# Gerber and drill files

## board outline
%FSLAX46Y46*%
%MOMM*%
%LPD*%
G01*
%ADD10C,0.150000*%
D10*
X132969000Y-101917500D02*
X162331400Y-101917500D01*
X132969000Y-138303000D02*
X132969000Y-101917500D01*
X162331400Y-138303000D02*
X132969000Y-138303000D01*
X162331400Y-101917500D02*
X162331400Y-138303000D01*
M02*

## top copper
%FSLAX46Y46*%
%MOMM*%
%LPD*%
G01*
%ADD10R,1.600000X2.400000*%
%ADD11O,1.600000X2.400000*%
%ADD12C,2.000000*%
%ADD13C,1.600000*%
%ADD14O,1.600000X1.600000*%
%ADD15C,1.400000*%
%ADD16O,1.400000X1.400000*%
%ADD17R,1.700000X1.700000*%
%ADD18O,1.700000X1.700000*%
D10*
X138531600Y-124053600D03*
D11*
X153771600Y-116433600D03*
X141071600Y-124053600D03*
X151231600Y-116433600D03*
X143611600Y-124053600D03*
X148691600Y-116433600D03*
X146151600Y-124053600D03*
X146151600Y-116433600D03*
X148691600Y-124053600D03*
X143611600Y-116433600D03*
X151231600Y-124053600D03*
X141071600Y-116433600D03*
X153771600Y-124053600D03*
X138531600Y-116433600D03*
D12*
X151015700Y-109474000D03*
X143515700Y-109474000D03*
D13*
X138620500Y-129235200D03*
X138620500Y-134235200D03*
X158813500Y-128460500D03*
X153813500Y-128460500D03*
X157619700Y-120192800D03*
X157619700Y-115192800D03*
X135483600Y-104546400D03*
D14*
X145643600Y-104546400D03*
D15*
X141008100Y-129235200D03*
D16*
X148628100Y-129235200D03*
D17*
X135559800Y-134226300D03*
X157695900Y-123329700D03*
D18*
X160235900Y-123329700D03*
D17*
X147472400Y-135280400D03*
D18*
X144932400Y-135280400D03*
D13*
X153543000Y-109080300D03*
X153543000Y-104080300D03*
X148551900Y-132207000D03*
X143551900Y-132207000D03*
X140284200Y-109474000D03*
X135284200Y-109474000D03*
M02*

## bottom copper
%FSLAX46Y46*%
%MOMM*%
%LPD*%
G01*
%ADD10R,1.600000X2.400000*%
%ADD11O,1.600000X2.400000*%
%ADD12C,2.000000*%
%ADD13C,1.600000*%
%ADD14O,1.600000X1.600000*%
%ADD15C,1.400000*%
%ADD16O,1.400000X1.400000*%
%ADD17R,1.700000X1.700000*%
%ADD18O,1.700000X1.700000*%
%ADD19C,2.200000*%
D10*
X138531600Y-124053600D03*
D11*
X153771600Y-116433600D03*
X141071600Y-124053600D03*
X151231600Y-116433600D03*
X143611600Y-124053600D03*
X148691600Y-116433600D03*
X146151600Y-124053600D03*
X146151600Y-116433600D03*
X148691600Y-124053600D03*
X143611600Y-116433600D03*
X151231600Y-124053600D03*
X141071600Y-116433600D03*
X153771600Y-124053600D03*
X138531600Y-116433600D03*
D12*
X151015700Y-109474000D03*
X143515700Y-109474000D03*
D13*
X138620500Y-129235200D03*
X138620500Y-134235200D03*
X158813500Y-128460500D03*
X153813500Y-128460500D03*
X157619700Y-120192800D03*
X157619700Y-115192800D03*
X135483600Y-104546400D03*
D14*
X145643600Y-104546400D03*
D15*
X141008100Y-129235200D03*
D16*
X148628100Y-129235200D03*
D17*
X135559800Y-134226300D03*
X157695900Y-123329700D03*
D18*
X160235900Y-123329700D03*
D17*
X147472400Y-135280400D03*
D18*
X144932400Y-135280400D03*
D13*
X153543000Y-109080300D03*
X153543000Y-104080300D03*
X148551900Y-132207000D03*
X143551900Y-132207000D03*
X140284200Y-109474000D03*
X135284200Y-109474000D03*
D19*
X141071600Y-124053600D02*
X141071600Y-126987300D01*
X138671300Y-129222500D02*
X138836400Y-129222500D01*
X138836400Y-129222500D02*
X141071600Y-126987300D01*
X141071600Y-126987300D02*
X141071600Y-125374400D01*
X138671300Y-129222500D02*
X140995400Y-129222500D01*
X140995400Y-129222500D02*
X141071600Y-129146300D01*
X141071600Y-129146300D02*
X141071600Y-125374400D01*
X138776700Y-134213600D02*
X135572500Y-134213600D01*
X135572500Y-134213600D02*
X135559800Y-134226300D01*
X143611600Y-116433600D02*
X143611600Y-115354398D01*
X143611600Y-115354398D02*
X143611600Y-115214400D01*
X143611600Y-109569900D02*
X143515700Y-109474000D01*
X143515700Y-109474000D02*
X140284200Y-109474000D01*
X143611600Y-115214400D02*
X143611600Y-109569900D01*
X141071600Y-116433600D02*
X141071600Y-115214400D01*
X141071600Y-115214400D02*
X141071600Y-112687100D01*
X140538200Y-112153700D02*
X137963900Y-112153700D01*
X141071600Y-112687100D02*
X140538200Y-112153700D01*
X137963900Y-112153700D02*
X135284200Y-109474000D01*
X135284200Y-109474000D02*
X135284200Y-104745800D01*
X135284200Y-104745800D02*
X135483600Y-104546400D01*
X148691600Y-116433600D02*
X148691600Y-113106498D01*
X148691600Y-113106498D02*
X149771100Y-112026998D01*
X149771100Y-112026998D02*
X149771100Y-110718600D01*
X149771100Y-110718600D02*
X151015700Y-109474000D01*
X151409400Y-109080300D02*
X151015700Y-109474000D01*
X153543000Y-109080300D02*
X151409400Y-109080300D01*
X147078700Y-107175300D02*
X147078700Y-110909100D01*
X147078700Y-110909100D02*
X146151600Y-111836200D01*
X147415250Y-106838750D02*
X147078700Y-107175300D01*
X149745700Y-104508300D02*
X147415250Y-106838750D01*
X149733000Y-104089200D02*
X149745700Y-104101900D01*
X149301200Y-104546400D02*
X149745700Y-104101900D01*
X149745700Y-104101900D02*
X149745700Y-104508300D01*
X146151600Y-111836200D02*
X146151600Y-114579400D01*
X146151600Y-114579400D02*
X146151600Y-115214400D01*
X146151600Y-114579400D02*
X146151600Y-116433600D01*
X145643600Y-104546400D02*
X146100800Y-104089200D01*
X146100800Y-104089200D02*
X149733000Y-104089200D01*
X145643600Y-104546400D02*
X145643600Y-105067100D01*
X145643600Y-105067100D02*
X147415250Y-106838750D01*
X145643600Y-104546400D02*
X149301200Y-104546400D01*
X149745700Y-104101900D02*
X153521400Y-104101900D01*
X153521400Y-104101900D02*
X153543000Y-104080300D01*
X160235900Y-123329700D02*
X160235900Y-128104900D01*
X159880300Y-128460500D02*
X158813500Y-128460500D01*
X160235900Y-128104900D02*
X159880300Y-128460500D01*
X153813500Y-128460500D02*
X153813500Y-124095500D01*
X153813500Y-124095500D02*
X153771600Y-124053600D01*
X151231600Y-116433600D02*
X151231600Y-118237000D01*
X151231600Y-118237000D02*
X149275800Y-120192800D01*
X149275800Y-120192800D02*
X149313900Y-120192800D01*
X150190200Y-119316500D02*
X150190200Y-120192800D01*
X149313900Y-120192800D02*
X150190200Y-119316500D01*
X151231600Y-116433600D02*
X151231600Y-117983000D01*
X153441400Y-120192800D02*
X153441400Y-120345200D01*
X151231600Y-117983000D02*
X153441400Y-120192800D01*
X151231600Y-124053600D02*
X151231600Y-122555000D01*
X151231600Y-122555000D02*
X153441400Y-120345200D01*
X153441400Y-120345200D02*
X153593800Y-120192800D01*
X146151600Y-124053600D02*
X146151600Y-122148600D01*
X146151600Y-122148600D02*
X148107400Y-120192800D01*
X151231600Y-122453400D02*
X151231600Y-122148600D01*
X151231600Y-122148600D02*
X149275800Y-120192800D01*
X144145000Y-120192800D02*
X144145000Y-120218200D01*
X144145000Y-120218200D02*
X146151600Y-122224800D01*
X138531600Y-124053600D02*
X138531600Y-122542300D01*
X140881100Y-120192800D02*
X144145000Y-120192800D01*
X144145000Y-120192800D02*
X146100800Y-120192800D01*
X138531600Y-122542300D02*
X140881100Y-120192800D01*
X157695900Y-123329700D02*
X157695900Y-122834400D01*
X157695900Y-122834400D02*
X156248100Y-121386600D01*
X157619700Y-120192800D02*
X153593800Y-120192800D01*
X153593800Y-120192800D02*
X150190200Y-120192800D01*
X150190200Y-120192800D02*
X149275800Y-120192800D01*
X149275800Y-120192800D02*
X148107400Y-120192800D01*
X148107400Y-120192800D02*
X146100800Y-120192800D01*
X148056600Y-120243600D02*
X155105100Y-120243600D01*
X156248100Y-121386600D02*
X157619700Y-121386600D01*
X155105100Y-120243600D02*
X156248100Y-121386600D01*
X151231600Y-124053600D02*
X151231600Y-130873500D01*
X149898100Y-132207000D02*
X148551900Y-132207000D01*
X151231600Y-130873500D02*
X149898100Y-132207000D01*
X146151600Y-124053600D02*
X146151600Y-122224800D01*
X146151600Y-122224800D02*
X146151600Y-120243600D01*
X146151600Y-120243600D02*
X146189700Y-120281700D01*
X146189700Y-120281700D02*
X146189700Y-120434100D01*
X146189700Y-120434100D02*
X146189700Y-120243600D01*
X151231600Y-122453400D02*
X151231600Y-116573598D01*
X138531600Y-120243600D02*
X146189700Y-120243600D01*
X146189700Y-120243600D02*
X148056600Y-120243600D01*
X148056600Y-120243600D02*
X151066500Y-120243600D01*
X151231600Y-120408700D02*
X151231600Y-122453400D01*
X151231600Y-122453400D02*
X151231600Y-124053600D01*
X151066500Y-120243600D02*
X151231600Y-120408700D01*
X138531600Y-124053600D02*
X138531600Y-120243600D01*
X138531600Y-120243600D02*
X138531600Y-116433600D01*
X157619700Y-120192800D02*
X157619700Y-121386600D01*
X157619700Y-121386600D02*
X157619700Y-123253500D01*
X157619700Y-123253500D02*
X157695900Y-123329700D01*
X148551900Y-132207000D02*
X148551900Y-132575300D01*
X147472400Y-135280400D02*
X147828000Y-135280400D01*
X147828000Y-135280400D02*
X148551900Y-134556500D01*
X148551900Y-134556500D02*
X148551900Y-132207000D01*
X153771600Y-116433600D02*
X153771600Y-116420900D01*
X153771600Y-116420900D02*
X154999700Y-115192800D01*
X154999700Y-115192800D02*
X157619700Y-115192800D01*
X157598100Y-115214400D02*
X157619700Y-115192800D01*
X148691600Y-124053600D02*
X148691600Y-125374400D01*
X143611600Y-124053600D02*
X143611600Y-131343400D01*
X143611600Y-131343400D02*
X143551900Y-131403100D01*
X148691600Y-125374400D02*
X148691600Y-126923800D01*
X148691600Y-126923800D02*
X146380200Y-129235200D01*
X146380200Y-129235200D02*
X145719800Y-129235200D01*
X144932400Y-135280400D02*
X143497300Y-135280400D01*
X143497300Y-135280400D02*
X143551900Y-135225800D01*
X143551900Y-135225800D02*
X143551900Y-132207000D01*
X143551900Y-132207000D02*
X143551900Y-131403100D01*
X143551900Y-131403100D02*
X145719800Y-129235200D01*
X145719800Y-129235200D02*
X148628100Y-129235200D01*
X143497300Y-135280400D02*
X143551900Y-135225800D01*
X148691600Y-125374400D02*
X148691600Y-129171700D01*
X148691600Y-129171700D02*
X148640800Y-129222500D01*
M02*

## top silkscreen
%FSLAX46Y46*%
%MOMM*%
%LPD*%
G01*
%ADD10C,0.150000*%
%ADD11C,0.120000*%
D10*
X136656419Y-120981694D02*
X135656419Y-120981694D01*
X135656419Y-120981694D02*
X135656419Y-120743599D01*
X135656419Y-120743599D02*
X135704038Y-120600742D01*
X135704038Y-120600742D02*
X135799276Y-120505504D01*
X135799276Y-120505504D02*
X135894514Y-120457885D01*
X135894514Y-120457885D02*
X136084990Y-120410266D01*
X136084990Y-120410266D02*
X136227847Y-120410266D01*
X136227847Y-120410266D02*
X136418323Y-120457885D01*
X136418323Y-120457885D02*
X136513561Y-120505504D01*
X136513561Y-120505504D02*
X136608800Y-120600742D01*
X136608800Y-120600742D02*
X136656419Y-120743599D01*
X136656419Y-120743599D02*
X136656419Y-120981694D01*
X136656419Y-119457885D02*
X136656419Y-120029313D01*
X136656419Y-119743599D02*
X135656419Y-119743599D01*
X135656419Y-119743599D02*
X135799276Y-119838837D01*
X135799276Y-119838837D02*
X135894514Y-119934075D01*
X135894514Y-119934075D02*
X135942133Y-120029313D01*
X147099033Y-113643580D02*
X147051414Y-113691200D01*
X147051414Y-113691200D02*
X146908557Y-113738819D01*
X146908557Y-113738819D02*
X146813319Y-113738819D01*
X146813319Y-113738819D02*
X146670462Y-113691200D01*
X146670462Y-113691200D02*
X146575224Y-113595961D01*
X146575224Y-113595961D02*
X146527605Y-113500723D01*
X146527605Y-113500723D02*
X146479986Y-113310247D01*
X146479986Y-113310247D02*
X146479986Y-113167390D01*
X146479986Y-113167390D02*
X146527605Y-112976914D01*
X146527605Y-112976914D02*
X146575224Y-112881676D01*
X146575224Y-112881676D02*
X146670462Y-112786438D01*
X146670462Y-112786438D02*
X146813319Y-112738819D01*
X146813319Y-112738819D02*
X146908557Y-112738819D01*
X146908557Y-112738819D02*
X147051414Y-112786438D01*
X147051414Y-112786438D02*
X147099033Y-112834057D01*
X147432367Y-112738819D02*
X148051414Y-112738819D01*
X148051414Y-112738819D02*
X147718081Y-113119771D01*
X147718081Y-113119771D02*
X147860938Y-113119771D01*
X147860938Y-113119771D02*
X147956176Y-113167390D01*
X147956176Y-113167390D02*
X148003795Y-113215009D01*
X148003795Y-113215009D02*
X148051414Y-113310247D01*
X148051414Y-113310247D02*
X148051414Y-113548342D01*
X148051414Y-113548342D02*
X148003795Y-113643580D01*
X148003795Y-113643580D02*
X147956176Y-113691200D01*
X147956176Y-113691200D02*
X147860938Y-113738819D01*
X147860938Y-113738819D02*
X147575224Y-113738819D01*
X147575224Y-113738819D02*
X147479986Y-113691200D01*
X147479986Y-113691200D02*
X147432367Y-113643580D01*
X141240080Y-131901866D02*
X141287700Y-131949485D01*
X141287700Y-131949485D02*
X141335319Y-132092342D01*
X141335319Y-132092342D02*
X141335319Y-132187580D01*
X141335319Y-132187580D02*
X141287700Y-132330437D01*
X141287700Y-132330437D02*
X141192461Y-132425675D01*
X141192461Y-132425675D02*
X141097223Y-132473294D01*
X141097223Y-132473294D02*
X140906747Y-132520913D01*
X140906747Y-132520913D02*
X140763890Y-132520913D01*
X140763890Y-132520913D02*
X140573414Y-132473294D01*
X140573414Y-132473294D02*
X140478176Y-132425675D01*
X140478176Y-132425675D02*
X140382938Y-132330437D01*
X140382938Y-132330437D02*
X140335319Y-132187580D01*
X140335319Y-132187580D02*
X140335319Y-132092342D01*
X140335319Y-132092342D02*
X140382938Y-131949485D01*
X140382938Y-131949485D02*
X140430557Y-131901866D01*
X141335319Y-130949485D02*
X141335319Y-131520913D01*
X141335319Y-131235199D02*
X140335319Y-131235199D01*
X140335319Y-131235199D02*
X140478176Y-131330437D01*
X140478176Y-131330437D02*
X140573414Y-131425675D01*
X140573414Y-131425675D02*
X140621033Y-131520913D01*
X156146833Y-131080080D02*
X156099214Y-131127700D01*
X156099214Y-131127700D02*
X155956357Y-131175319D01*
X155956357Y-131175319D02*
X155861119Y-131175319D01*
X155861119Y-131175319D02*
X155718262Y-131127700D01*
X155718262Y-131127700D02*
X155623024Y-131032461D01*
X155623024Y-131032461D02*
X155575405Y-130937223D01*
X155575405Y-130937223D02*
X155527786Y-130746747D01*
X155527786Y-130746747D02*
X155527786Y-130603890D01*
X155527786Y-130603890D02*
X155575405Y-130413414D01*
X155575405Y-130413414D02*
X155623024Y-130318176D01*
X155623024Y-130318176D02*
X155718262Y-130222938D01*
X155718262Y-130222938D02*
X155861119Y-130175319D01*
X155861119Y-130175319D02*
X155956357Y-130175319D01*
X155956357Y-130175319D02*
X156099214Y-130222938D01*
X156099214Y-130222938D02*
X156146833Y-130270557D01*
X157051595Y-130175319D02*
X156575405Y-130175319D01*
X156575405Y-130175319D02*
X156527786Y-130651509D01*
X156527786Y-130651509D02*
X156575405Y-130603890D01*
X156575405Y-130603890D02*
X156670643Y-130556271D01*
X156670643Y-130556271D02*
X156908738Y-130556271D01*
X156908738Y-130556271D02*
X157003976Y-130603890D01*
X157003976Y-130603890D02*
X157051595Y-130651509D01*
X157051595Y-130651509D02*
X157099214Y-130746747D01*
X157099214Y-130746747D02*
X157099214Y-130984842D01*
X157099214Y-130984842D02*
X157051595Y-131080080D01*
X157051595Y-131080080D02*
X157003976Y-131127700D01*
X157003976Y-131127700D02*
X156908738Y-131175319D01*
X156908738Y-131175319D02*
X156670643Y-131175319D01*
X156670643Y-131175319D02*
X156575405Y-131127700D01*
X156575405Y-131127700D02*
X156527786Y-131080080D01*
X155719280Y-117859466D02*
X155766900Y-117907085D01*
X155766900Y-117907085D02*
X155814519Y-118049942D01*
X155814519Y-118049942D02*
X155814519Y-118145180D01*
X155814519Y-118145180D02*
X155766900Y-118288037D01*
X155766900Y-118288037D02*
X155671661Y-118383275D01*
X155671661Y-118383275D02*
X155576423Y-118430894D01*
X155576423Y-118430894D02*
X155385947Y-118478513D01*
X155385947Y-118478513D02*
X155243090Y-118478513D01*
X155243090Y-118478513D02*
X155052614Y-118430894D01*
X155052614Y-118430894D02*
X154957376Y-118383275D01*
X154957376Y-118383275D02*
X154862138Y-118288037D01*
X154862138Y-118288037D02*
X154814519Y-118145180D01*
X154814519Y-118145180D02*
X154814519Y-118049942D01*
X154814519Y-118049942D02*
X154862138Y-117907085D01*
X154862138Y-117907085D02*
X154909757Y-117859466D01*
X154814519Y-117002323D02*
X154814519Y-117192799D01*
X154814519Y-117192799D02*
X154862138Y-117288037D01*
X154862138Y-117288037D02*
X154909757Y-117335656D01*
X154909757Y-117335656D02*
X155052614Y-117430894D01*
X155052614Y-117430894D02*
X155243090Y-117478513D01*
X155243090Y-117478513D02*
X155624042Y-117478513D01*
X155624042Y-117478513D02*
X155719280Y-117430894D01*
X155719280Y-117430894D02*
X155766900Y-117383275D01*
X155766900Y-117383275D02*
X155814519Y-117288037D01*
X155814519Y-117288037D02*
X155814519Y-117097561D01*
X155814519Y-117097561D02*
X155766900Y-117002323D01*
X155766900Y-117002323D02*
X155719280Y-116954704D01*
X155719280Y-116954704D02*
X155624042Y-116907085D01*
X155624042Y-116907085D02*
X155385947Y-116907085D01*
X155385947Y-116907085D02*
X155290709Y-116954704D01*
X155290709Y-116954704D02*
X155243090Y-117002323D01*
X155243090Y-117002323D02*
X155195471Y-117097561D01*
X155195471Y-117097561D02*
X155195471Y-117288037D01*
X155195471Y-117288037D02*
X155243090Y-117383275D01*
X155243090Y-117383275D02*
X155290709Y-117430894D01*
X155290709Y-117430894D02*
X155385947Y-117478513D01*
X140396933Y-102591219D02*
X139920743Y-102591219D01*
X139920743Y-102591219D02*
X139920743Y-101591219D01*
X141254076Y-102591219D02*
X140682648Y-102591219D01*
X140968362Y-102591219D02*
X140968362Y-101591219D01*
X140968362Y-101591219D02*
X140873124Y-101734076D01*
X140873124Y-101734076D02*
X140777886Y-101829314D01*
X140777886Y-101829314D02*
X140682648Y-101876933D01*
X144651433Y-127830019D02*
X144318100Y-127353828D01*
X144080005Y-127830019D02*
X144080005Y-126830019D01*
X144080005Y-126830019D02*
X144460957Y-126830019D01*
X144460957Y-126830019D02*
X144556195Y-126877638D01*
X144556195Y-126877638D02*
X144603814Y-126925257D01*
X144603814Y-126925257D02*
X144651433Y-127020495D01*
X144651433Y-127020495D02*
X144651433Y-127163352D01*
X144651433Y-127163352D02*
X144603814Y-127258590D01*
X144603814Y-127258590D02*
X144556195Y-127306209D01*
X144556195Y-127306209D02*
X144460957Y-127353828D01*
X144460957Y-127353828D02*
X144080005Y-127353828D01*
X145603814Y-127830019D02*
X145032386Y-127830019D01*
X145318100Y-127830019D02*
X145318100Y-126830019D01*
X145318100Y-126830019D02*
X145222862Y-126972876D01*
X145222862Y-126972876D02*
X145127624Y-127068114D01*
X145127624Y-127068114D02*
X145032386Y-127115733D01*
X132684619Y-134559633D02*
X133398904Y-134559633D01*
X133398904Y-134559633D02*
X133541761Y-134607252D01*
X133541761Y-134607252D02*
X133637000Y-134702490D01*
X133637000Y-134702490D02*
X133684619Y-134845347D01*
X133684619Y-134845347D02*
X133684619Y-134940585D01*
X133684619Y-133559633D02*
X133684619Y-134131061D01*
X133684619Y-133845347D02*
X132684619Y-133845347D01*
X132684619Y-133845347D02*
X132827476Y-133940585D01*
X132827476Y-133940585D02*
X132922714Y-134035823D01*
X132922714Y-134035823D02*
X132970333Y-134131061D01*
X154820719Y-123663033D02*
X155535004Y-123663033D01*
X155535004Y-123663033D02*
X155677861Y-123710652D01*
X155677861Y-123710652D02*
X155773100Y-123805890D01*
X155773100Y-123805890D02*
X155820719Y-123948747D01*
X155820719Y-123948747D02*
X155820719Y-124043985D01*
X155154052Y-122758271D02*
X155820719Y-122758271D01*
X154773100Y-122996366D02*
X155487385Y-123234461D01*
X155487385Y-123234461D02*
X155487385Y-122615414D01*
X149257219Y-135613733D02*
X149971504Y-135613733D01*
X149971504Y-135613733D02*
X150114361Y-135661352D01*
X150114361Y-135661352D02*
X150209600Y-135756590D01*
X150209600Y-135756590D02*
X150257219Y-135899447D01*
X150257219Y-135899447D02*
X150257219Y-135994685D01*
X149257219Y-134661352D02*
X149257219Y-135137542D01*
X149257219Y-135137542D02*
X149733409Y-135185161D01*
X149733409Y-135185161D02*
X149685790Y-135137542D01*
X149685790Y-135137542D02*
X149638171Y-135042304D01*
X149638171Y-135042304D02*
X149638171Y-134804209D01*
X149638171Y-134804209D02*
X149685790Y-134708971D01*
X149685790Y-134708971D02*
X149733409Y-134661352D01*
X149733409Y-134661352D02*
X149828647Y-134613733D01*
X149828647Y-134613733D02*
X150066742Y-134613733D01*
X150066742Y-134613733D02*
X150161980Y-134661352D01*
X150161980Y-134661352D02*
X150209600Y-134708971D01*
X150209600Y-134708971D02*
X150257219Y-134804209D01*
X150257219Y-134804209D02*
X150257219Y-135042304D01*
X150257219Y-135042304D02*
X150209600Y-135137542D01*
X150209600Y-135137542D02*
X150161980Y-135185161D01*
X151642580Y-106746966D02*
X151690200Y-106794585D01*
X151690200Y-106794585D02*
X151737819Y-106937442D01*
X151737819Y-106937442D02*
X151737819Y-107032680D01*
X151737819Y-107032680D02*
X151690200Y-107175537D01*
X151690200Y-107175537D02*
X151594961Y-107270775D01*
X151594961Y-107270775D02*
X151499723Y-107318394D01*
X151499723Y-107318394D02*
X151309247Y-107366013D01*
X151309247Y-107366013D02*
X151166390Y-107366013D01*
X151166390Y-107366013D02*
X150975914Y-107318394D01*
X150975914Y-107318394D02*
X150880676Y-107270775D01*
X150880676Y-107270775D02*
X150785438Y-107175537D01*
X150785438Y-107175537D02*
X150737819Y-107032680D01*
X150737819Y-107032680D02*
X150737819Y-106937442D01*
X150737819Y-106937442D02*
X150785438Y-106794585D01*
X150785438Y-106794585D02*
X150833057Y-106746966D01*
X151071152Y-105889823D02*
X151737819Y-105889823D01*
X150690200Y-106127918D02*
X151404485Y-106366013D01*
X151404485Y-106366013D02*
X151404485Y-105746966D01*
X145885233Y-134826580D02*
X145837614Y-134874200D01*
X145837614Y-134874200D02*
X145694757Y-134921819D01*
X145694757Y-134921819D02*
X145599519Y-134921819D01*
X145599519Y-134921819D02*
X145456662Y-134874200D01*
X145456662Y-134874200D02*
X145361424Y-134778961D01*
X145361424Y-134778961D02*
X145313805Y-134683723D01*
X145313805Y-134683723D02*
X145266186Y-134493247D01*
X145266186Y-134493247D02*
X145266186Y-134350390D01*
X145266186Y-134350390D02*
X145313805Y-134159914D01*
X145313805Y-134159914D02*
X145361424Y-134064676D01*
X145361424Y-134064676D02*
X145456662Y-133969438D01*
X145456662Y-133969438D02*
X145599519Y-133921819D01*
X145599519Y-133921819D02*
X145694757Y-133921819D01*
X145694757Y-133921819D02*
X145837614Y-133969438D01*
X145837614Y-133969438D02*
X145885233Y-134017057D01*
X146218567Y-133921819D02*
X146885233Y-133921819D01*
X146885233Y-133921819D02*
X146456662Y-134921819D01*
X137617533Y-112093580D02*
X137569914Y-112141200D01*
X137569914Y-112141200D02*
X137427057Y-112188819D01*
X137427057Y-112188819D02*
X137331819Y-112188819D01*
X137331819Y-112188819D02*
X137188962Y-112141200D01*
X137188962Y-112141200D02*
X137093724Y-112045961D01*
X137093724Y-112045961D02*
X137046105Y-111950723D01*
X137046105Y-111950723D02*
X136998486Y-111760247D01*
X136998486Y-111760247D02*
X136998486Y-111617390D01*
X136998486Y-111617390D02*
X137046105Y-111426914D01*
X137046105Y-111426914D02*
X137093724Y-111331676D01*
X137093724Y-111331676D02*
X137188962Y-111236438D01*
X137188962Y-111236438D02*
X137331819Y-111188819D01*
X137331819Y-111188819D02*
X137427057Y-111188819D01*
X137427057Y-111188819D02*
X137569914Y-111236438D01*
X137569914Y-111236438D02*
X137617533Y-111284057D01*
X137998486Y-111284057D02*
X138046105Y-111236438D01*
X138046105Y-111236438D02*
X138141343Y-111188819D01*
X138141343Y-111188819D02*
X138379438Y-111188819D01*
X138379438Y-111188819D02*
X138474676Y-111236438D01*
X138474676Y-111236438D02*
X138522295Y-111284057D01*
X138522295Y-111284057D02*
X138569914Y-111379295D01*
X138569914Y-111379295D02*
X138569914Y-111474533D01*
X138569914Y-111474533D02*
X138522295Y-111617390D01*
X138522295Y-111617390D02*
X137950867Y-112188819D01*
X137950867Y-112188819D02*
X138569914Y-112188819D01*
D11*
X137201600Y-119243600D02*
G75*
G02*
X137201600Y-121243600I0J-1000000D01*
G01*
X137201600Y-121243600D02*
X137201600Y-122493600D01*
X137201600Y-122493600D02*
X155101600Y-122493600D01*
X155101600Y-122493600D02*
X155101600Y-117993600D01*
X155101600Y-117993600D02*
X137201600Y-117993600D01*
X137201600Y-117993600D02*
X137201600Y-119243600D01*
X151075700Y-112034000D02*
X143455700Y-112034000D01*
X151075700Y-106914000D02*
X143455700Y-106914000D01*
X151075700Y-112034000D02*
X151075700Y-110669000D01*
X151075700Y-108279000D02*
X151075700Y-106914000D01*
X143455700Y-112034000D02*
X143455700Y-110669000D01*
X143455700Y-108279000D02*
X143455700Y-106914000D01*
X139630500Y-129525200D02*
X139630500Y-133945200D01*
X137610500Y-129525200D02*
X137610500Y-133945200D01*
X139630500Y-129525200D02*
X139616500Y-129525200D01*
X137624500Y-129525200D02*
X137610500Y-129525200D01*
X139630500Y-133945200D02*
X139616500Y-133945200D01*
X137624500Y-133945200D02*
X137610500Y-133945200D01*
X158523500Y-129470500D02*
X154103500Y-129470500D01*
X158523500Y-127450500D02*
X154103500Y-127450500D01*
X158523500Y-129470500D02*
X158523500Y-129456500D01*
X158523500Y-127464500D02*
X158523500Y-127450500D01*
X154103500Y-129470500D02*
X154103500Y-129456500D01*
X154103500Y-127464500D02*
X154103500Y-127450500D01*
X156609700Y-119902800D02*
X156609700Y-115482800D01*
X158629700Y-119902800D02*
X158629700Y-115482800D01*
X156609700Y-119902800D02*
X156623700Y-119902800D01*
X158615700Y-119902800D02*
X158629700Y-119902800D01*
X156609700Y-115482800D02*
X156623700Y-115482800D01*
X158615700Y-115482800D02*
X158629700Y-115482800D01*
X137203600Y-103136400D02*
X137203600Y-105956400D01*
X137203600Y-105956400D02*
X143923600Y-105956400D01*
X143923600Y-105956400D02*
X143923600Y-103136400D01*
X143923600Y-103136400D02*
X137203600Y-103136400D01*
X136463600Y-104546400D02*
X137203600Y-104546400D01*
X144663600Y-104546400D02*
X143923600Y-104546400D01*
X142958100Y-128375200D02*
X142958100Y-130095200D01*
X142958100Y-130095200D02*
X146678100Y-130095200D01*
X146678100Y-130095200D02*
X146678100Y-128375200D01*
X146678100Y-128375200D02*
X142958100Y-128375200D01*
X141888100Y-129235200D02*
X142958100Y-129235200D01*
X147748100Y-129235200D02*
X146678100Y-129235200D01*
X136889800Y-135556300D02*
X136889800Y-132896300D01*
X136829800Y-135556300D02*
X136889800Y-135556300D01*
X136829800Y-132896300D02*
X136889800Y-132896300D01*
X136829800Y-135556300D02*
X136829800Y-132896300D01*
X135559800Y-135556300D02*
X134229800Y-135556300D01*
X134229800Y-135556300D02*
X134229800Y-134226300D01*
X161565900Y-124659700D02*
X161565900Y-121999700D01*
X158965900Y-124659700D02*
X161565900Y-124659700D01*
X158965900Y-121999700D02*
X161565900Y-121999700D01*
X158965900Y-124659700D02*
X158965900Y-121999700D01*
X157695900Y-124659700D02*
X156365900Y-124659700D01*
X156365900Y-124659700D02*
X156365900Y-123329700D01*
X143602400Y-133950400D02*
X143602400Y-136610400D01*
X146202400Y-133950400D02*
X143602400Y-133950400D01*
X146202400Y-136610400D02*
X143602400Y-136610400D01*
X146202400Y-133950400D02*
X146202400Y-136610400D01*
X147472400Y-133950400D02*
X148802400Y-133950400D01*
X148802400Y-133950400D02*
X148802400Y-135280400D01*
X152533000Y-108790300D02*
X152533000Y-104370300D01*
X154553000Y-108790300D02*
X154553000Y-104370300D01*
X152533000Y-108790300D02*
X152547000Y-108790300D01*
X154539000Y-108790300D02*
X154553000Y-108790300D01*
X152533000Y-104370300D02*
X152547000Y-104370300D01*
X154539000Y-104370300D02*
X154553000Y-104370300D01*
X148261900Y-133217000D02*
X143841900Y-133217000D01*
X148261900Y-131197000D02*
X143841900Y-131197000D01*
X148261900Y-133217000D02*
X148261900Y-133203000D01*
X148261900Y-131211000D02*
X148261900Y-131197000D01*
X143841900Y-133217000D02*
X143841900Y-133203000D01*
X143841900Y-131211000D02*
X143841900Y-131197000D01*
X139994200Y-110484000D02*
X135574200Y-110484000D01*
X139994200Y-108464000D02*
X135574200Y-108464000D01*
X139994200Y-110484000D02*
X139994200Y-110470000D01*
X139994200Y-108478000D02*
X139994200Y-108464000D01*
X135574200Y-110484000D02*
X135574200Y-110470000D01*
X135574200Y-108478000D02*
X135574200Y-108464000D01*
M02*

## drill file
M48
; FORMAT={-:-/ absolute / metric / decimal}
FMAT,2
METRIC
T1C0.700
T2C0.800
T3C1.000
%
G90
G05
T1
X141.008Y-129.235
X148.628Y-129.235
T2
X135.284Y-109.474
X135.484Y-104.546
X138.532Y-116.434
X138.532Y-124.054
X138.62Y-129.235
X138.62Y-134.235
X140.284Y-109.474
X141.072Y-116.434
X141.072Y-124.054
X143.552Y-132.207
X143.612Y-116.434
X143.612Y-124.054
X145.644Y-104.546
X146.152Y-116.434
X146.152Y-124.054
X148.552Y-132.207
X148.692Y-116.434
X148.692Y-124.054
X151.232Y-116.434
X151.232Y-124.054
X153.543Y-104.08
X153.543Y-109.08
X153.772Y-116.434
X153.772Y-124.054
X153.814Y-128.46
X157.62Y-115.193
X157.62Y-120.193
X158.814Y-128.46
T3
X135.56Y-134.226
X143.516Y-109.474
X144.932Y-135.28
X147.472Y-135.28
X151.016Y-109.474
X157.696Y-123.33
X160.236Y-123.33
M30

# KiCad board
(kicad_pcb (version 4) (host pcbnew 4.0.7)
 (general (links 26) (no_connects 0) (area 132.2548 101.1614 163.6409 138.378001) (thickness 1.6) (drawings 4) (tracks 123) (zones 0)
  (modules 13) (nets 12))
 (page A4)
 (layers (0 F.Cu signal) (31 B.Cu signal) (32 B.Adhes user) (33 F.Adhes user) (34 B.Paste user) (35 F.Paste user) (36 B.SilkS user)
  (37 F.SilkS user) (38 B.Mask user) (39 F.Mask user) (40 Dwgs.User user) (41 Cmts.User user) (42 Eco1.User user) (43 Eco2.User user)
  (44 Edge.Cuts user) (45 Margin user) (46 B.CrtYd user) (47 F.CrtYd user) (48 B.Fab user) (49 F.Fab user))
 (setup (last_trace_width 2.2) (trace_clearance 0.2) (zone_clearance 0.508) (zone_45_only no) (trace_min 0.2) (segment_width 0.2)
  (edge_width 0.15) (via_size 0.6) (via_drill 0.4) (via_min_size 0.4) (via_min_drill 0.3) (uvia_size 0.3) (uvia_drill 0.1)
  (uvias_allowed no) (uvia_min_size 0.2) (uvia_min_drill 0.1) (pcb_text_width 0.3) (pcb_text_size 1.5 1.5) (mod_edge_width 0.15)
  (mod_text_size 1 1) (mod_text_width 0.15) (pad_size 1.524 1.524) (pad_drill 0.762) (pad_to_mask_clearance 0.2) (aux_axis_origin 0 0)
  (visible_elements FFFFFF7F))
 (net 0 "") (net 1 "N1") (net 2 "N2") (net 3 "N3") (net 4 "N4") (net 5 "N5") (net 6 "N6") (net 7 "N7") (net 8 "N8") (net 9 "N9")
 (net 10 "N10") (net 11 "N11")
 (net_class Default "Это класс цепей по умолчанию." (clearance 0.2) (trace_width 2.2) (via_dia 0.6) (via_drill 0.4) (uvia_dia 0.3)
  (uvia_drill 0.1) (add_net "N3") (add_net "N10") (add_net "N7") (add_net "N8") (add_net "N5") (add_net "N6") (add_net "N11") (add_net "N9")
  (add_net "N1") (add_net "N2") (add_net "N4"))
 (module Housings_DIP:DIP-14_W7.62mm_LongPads (layer F.Cu) (at 138.5316 124.0536 90)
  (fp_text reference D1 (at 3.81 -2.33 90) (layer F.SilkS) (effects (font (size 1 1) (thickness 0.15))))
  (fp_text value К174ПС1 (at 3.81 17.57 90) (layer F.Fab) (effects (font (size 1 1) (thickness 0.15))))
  (fp_arc (start 3.81 -1.33) (end 2.81 -1.33) (angle -180) (layer F.SilkS) (width 0.12))
  (fp_line (start 2.81 -1.33) (end 1.56 -1.33) (layer F.SilkS) (width 0.12))
  (fp_line (start 1.56 -1.33) (end 1.56 16.57) (layer F.SilkS) (width 0.12))
  (fp_line (start 1.56 16.57) (end 6.06 16.57) (layer F.SilkS) (width 0.12))
  (fp_line (start 6.06 16.57) (end 6.06 -1.33) (layer F.SilkS) (width 0.12))
  (fp_line (start 6.06 -1.33) (end 4.81 -1.33) (layer F.SilkS) (width 0.12))
  (pad 1 thru_hole rect (at 0 0 90) (size 2.4 1.6) (drill 0.8) (layers *.Cu *.Mask) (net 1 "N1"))
  (pad 8 thru_hole oval (at 7.62 15.24 90) (size 2.4 1.6) (drill 0.8) (layers *.Cu *.Mask) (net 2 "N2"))
  (pad 2 thru_hole oval (at 0 2.54 90) (size 2.4 1.6) (drill 0.8) (layers *.Cu *.Mask) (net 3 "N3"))
  (pad 9 thru_hole oval (at 7.62 12.7 90) (size 2.4 1.6) (drill 0.8) (layers *.Cu *.Mask) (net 1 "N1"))
  (pad 3 thru_hole oval (at 0 5.08 90) (size 2.4 1.6) (drill 0.8) (layers *.Cu *.Mask) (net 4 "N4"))
  (pad 10 thru_hole oval (at 7.62 10.16 90) (size 2.4 1.6) (drill 0.8) (layers *.Cu *.Mask) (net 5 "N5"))
  (pad 4 thru_hole oval (at 0 7.62 90) (size 2.4 1.6) (drill 0.8) (layers *.Cu *.Mask) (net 1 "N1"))
  (pad 11 thru_hole oval (at 7.62 7.62 90) (size 2.4 1.6) (drill 0.8) (layers *.Cu *.Mask) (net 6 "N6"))
  (pad 5 thru_hole oval (at 0 10.16 90) (size 2.4 1.6) (drill 0.8) (layers *.Cu *.Mask) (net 4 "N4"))
  (pad 12 thru_hole oval (at 7.62 5.08 90) (size 2.4 1.6) (drill 0.8) (layers *.Cu *.Mask) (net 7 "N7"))
  (pad 6 thru_hole oval (at 0 12.7 90) (size 2.4 1.6) (drill 0.8) (layers *.Cu *.Mask) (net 1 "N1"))
  (pad 13 thru_hole oval (at 7.62 2.54 90) (size 2.4 1.6) (drill 0.8) (layers *.Cu *.Mask) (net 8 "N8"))
  (pad 7 thru_hole oval (at 0 15.24 90) (size 2.4 1.6) (drill 0.8) (layers *.Cu *.Mask) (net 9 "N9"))
  (pad 14 thru_hole oval (at 7.62 0 90) (size 2.4 1.6) (drill 0.8) (layers *.Cu *.Mask) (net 1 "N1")))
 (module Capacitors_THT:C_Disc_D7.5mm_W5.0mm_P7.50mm (layer F.Cu) (at 151.0157 109.474 180)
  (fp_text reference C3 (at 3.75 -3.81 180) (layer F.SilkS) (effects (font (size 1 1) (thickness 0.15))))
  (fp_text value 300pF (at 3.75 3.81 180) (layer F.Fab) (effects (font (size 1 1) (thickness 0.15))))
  (fp_line (start -0.06 -2.56) (end 7.56 -2.56) (layer F.SilkS) (width 0.12))
  (fp_line (start -0.06 2.56) (end 7.56 2.56) (layer F.SilkS) (width 0.12))
  (fp_line (start -0.06 -2.56) (end -0.06 -1.195) (layer F.SilkS) (width 0.12))
  (fp_line (start -0.06 1.195) (end -0.06 2.56) (layer F.SilkS) (width 0.12))
  (fp_line (start 7.56 -2.56) (end 7.56 -1.195) (layer F.SilkS) (width 0.12))
  (fp_line (start 7.56 1.195) (end 7.56 2.56) (layer F.SilkS) (width 0.12))
  (pad 1 thru_hole circle (at 0 0 180) (size 2 2) (drill 1) (layers *.Cu *.Mask) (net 5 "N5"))
  (pad 2 thru_hole circle (at 7.5 0 180) (size 2 2) (drill 1) (layers *.Cu *.Mask) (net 7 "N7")))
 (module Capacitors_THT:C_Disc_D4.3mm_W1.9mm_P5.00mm (layer F.Cu) (at 138.6205 129.2352 270)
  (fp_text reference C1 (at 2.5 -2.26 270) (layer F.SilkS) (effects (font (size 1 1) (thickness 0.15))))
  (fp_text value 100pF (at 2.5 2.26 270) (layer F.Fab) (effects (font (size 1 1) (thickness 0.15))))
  (fp_line (start 0.29 -1.01) (end 4.71 -1.01) (layer F.SilkS) (width 0.12))
  (fp_line (start 0.29 1.01) (end 4.71 1.01) (layer F.SilkS) (width 0.12))
  (fp_line (start 0.29 -1.01) (end 0.29 -0.996) (layer F.SilkS) (width 0.12))
  (fp_line (start 0.29 0.996) (end 0.29 1.01) (layer F.SilkS) (width 0.12))
  (fp_line (start 4.71 -1.01) (end 4.71 -0.996) (layer F.SilkS) (width 0.12))
  (fp_line (start 4.71 0.996) (end 4.71 1.01) (layer F.SilkS) (width 0.12))
  (pad 1 thru_hole circle (at 0 0 270) (size 1.6 1.6) (drill 0.8) (layers *.Cu *.Mask) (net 3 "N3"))
  (pad 2 thru_hole circle (at 5 0 270) (size 1.6 1.6) (drill 0.8) (layers *.Cu *.Mask) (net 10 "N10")))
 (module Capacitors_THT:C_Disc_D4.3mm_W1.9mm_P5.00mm (layer F.Cu) (at 158.8135 128.4605 180)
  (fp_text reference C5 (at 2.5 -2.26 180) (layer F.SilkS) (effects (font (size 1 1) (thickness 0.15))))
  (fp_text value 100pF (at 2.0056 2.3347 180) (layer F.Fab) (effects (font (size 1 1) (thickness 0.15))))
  (fp_line (start 0.29 -1.01) (end 4.71 -1.01) (layer F.SilkS) (width 0.12))
  (fp_line (start 0.29 1.01) (end 4.71 1.01) (layer F.SilkS) (width 0.12))
  (fp_line (start 0.29 -1.01) (end 0.29 -0.996) (layer F.SilkS) (width 0.12))
  (fp_line (start 0.29 0.996) (end 0.29 1.01) (layer F.SilkS) (width 0.12))
  (fp_line (start 4.71 -1.01) (end 4.71 -0.996) (layer F.SilkS) (width 0.12))
  (fp_line (start 4.71 0.996) (end 4.71 1.01) (layer F.SilkS) (width 0.12))
  (pad 1 thru_hole circle (at 0 0 180) (size 1.6 1.6) (drill 0.8) (layers *.Cu *.Mask) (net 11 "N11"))
  (pad 2 thru_hole circle (at 5 0 180) (size 1.6 1.6) (drill 0.8) (layers *.Cu *.Mask) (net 9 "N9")))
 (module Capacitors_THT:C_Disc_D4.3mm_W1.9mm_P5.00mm (layer F.Cu) (at 157.6197 120.1928 90)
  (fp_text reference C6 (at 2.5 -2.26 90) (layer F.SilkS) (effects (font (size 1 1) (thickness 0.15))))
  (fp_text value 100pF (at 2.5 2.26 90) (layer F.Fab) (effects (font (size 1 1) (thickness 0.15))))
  (fp_line (start 0.29 -1.01) (end 4.71 -1.01) (layer F.SilkS) (width 0.12))
  (fp_line (start 0.29 1.01) (end 4.71 1.01) (layer F.SilkS) (width 0.12))
  (fp_line (start 0.29 -1.01) (end 0.29 -0.996) (layer F.SilkS) (width 0.12))
  (fp_line (start 0.29 0.996) (end 0.29 1.01) (layer F.SilkS) (width 0.12))
  (fp_line (start 4.71 -1.01) (end 4.71 -0.996) (layer F.SilkS) (width 0.12))
  (fp_line (start 4.71 0.996) (end 4.71 1.01) (layer F.SilkS) (width 0.12))
  (pad 1 thru_hole circle (at 0 0 90) (size 1.6 1.6) (drill 0.8) (layers *.Cu *.Mask) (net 1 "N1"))
  (pad 2 thru_hole circle (at 5 0 90) (size 1.6 1.6) (drill 0.8) (layers *.Cu *.Mask) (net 2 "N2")))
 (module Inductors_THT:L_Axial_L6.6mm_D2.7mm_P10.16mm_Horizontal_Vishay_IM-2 (layer F.Cu) (at 135.4836 104.5464)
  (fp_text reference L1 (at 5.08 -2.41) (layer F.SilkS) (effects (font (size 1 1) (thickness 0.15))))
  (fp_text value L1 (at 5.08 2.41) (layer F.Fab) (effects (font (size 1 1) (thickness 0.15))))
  (fp_line (start 1.72 -1.41) (end 1.72 1.41) (layer F.SilkS) (width 0.12))
  (fp_line (start 1.72 1.41) (end 8.44 1.41) (layer F.SilkS) (width 0.12))
  (fp_line (start 8.44 1.41) (end 8.44 -1.41) (layer F.SilkS) (width 0.12))
  (fp_line (start 8.44 -1.41) (end 1.72 -1.41) (layer F.SilkS) (width 0.12))
  (fp_line (start 0.98 0) (end 1.72 0) (layer F.SilkS) (width 0.12))
  (fp_line (start 9.18 0) (end 8.44 0) (layer F.SilkS) (width 0.12))
  (pad 1 thru_hole circle (at 0 0) (size 1.6 1.6) (drill 0.8) (layers *.Cu *.Mask) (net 8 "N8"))
  (pad 2 thru_hole oval (at 10.16 0) (size 1.6 1.6) (drill 0.8) (layers *.Cu *.Mask) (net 6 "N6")))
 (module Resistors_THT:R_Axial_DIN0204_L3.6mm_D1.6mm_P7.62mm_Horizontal (layer F.Cu) (at 141.0081 129.2352)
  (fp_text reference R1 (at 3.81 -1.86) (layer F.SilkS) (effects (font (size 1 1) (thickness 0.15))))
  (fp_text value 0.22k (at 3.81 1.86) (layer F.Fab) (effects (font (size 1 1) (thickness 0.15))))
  (fp_line (start 1.95 -0.86) (end 1.95 0.86) (layer F.SilkS) (width 0.12))
  (fp_line (start 1.95 0.86) (end 5.67 0.86) (layer F.SilkS) (width 0.12))
  (fp_line (start 5.67 0.86) (end 5.67 -0.86) (layer F.SilkS) (width 0.12))
  (fp_line (start 5.67 -0.86) (end 1.95 -0.86) (layer F.SilkS) (width 0.12))
  (fp_line (start 0.88 0) (end 1.95 0) (layer F.SilkS) (width 0.12))
  (fp_line (start 6.74 0) (end 5.67 0) (layer F.SilkS) (width 0.12))
  (pad 1 thru_hole circle (at 0 0) (size 1.4 1.4) (drill 0.7) (layers *.Cu *.Mask) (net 3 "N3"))
  (pad 2 thru_hole oval (at 7.62 0) (size 1.4 1.4) (drill 0.7) (layers *.Cu *.Mask) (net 4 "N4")))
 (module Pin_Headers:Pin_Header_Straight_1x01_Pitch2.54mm (layer F.Cu) (at 135.5598 134.2263 90)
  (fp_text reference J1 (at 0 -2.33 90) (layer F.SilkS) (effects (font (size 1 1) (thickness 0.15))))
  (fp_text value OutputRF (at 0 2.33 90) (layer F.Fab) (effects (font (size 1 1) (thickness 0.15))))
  (fp_line (start -1.33 1.33) (end 1.33 1.33) (layer F.SilkS) (width 0.12))
  (fp_line (start -1.33 1.27) (end -1.33 1.33) (layer F.SilkS) (width 0.12))
  (fp_line (start 1.33 1.27) (end 1.33 1.33) (layer F.SilkS) (width 0.12))
  (fp_line (start -1.33 1.27) (end 1.33 1.27) (layer F.SilkS) (width 0.12))
  (fp_line (start -1.33 0) (end -1.33 -1.33) (layer F.SilkS) (width 0.12))
  (fp_line (start -1.33 -1.33) (end 0 -1.33) (layer F.SilkS) (width 0.12))
  (pad 1 thru_hole rect (at 0 0 90) (size 1.7 1.7) (drill 1) (layers *.Cu *.Mask) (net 10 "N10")))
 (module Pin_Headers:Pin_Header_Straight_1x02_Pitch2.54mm (layer F.Cu) (at 157.6959 123.3297 90)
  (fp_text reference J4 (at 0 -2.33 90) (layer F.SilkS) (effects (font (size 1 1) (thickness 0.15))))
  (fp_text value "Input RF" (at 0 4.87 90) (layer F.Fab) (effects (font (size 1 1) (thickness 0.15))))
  (fp_line (start -1.33 3.87) (end 1.33 3.87) (layer F.SilkS) (width 0.12))
  (fp_line (start -1.33 1.27) (end -1.33 3.87) (layer F.SilkS) (width 0.12))
  (fp_line (start 1.33 1.27) (end 1.33 3.87) (layer F.SilkS) (width 0.12))
  (fp_line (start -1.33 1.27) (end 1.33 1.27) (layer F.SilkS) (width 0.12))
  (fp_line (start -1.33 0) (end -1.33 -1.33) (layer F.SilkS) (width 0.12))
  (fp_line (start -1.33 -1.33) (end 0 -1.33) (layer F.SilkS) (width 0.12))
  (pad 1 thru_hole rect (at 0 0 90) (size 1.7 1.7) (drill 1) (layers *.Cu *.Mask) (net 1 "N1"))
  (pad 2 thru_hole oval (at 0 2.54 90) (size 1.7 1.7) (drill 1) (layers *.Cu *.Mask) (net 11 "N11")))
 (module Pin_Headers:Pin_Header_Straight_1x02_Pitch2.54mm (layer F.Cu) (at 147.4724 135.2804 270)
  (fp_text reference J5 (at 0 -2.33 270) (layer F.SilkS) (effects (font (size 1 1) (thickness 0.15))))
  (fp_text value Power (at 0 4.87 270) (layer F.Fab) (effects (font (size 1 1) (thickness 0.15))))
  (fp_line (start -1.33 3.87) (end 1.33 3.87) (layer F.SilkS) (width 0.12))
  (fp_line (start -1.33 1.27) (end -1.33 3.87) (layer F.SilkS) (width 0.12))
  (fp_line (start 1.33 1.27) (end 1.33 3.87) (layer F.SilkS) (width 0.12))
  (fp_line (start -1.33 1.27) (end 1.33 1.27) (layer F.SilkS) (width 0.12))
  (fp_line (start -1.33 0) (end -1.33 -1.33) (layer F.SilkS) (width 0.12))
  (fp_line (start -1.33 -1.33) (end 0 -1.33) (layer F.SilkS) (width 0.12))
  (pad 1 thru_hole rect (at 0 0 270) (size 1.7 1.7) (drill 1) (layers *.Cu *.Mask) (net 1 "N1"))
  (pad 2 thru_hole oval (at 0 2.54 270) (size 1.7 1.7) (drill 1) (layers *.Cu *.Mask) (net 4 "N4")))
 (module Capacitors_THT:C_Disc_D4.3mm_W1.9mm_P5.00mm (layer F.Cu) (at 153.543 109.0803 90)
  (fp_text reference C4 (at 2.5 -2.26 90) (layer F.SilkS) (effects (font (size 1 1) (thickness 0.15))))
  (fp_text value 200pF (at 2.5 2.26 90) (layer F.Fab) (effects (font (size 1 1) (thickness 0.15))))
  (fp_line (start 0.29 -1.01) (end 4.71 -1.01) (layer F.SilkS) (width 0.12))
  (fp_line (start 0.29 1.01) (end 4.71 1.01) (layer F.SilkS) (width 0.12))
  (fp_line (start 0.29 -1.01) (end 0.29 -0.996) (layer F.SilkS) (width 0.12))
  (fp_line (start 0.29 0.996) (end 0.29 1.01) (layer F.SilkS) (width 0.12))
  (fp_line (start 4.71 -1.01) (end 4.71 -0.996) (layer F.SilkS) (width 0.12))
  (fp_line (start 4.71 0.996) (end 4.71 1.01) (layer F.SilkS) (width 0.12))
  (pad 1 thru_hole circle (at 0 0 90) (size 1.6 1.6) (drill 0.8) (layers *.Cu *.Mask) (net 5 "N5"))
  (pad 2 thru_hole circle (at 5 0 90) (size 1.6 1.6) (drill 0.8) (layers *.Cu *.Mask) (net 6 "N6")))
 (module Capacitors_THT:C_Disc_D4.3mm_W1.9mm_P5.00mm (layer F.Cu) (at 148.5519 132.207 180)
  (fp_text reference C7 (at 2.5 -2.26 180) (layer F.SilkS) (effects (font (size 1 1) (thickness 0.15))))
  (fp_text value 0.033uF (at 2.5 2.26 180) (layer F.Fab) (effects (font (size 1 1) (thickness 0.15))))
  (fp_line (start 0.29 -1.01) (end 4.71 -1.01) (layer F.SilkS) (width 0.12))
  (fp_line (start 0.29 1.01) (end 4.71 1.01) (layer F.SilkS) (width 0.12))
  (fp_line (start 0.29 -1.01) (end 0.29 -0.996) (layer F.SilkS) (width 0.12))
  (fp_line (start 0.29 0.996) (end 0.29 1.01) (layer F.SilkS) (width 0.12))
  (fp_line (start 4.71 -1.01) (end 4.71 -0.996) (layer F.SilkS) (width 0.12))
  (fp_line (start 4.71 0.996) (end 4.71 1.01) (layer F.SilkS) (width 0.12))
  (pad 1 thru_hole circle (at 0 0 180) (size 1.6 1.6) (drill 0.8) (layers *.Cu *.Mask) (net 1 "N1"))
  (pad 2 thru_hole circle (at 5 0 180) (size 1.6 1.6) (drill 0.8) (layers *.Cu *.Mask) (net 4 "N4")))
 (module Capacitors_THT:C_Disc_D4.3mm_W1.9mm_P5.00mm (layer F.Cu) (at 140.2842 109.474 180)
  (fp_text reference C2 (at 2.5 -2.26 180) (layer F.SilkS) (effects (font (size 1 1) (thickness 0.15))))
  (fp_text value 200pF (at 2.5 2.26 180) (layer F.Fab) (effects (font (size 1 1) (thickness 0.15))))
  (fp_line (start 0.29 -1.01) (end 4.71 -1.01) (layer F.SilkS) (width 0.12))
  (fp_line (start 0.29 1.01) (end 4.71 1.01) (layer F.SilkS) (width 0.12))
  (fp_line (start 0.29 -1.01) (end 0.29 -0.996) (layer F.SilkS) (width 0.12))
  (fp_line (start 0.29 0.996) (end 0.29 1.01) (layer F.SilkS) (width 0.12))
  (fp_line (start 4.71 -1.01) (end 4.71 -0.996) (layer F.SilkS) (width 0.12))
  (fp_line (start 4.71 0.996) (end 4.71 1.01) (layer F.SilkS) (width 0.12))
  (pad 1 thru_hole circle (at 0 0 180) (size 1.6 1.6) (drill 0.8) (layers *.Cu *.Mask) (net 7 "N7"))
  (pad 2 thru_hole circle (at 5 0 180) (size 1.6 1.6) (drill 0.8) (layers *.Cu *.Mask) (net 8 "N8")))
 (gr_line (start 132.969 101.9175) (end 162.3314 101.9175) (angle 90) (layer Edge.Cuts) (width 0.15))
 (gr_line (start 132.969 138.303) (end 132.969 101.9175) (angle 90) (layer Edge.Cuts) (width 0.15))
 (gr_line (start 162.3314 138.303) (end 132.969 138.303) (angle 90) (layer Edge.Cuts) (width 0.15))
 (gr_line (start 162.3314 101.9175) (end 162.3314 138.303) (angle 90) (layer Edge.Cuts) (width 0.15))
 (segment (start 141.0716 124.0536) (end 141.0716 126.9873) (width 2.2) (layer B.Cu) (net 3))
 (segment (start 138.6713 129.2225) (end 138.8364 129.2225) (width 2.2) (layer B.Cu) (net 3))
 (segment (start 138.8364 129.2225) (end 141.0716 126.9873) (width 2.2) (layer B.Cu) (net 3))
 (segment (start 141.0716 126.9873) (end 141.0716 125.3744) (width 2.2) (layer B.Cu) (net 3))
 (segment (start 138.6713 129.2225) (end 140.9954 129.2225) (width 2.2) (layer B.Cu) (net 3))
 (segment (start 140.9954 129.2225) (end 141.0716 129.1463) (width 2.2) (layer B.Cu) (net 3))
 (segment (start 141.0716 129.1463) (end 141.0716 125.3744) (width 2.2) (layer B.Cu) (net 3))
 (segment (start 138.7767 134.2136) (end 135.5725 134.2136) (width 2.2) (layer B.Cu) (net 10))
 (segment (start 135.5725 134.2136) (end 135.5598 134.2263) (width 2.2) (layer B.Cu) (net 10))
 (segment (start 143.6116 116.4336) (end 143.6116 115.354398) (width 2.2) (layer B.Cu) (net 7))
 (segment (start 143.6116 115.354398) (end 143.6116 115.2144) (width 2.2) (layer B.Cu) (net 7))
 (segment (start 143.6116 109.5699) (end 143.5157 109.474) (width 2.2) (layer B.Cu) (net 7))
 (segment (start 143.5157 109.474) (end 140.2842 109.474) (width 2.2) (layer B.Cu) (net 7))
 (segment (start 143.6116 115.2144) (end 143.6116 109.5699) (width 2.2) (layer B.Cu) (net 7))
 (segment (start 141.0716 116.4336) (end 141.0716 115.2144) (width 2.2) (layer B.Cu) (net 8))
 (segment (start 141.0716 115.2144) (end 141.0716 112.6871) (width 2.2) (layer B.Cu) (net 8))
 (segment (start 140.5382 112.1537) (end 137.9639 112.1537) (width 2.2) (layer B.Cu) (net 8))
 (segment (start 141.0716 112.6871) (end 140.5382 112.1537) (width 2.2) (layer B.Cu) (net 8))
 (segment (start 137.9639 112.1537) (end 135.2842 109.474) (width 2.2) (layer B.Cu) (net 8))
 (segment (start 135.2842 109.474) (end 135.2842 104.7458) (width 2.2) (layer B.Cu) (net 8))
 (segment (start 135.2842 104.7458) (end 135.4836 104.5464) (width 2.2) (layer B.Cu) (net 8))
 (segment (start 148.6916 116.4336) (end 148.6916 113.106498) (width 2.2) (layer B.Cu) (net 5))
 (segment (start 148.6916 113.106498) (end 149.7711 112.026998) (width 2.2) (layer B.Cu) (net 5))
 (segment (start 149.7711 112.026998) (end 149.7711 110.7186) (width 2.2) (layer B.Cu) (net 5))
 (segment (start 149.7711 110.7186) (end 151.0157 109.474) (width 2.2) (layer B.Cu) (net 5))
 (segment (start 151.4094 109.0803) (end 151.0157 109.474) (width 2.2) (layer B.Cu) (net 5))
 (segment (start 153.543 109.0803) (end 151.4094 109.0803) (width 2.2) (layer B.Cu) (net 5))
 (segment (start 147.0787 107.1753) (end 147.0787 110.9091) (width 2.2) (layer B.Cu) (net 6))
 (segment (start 147.0787 110.9091) (end 146.1516 111.8362) (width 2.2) (layer B.Cu) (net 6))
 (segment (start 147.41525 106.83875) (end 147.0787 107.1753) (width 2.2) (layer B.Cu) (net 6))
 (segment (start 149.7457 104.5083) (end 147.41525 106.83875) (width 2.2) (layer B.Cu) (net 6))
 (segment (start 149.733 104.0892) (end 149.7457 104.1019) (width 2.2) (layer B.Cu) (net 6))
 (segment (start 149.3012 104.5464) (end 149.7457 104.1019) (width 2.2) (layer B.Cu) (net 6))
 (segment (start 149.7457 104.1019) (end 149.7457 104.5083) (width 2.2) (layer B.Cu) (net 6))
 (segment (start 146.1516 111.8362) (end 146.1516 114.5794) (width 2.2) (layer B.Cu) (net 6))
 (segment (start 146.1516 114.5794) (end 146.1516 115.2144) (width 2.2) (layer B.Cu) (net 6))
 (segment (start 146.1516 114.5794) (end 146.1516 116.4336) (width 2.2) (layer B.Cu) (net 6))
 (segment (start 145.6436 104.5464) (end 146.1008 104.0892) (width 2.2) (layer B.Cu) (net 6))
 (segment (start 146.1008 104.0892) (end 149.733 104.0892) (width 2.2) (layer B.Cu) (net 6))
 (segment (start 145.6436 104.5464) (end 145.6436 105.0671) (width 2.2) (layer B.Cu) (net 6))
 (segment (start 145.6436 105.0671) (end 147.41525 106.83875) (width 2.2) (layer B.Cu) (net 6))
 (segment (start 145.6436 104.5464) (end 149.3012 104.5464) (width 2.2) (layer B.Cu) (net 6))
 (segment (start 149.7457 104.1019) (end 153.5214 104.1019) (width 2.2) (layer B.Cu) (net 6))
 (segment (start 153.5214 104.1019) (end 153.543 104.0803) (width 2.2) (layer B.Cu) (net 6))
 (segment (start 160.2359 123.3297) (end 160.2359 128.1049) (width 2.2) (layer B.Cu) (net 11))
 (segment (start 159.8803 128.4605) (end 158.8135 128.4605) (width 2.2) (layer B.Cu) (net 11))
 (segment (start 160.2359 128.1049) (end 159.8803 128.4605) (width 2.2) (layer B.Cu) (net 11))
 (segment (start 153.8135 128.4605) (end 153.8135 124.0955) (width 2.2) (layer B.Cu) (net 9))
 (segment (start 153.8135 124.0955) (end 153.7716 124.0536) (width 2.2) (layer B.Cu) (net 9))
 (segment (start 151.2316 116.4336) (end 151.2316 118.237) (width 2.2) (layer B.Cu) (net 1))
 (segment (start 151.2316 118.237) (end 149.2758 120.1928) (width 2.2) (layer B.Cu) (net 1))
 (segment (start 149.2758 120.1928) (end 149.3139 120.1928) (width 2.2) (layer B.Cu) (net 1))
 (segment (start 150.1902 119.3165) (end 150.1902 120.1928) (width 2.2) (layer B.Cu) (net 1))
 (segment (start 149.3139 120.1928) (end 150.1902 119.3165) (width 2.2) (layer B.Cu) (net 1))
 (segment (start 151.2316 116.4336) (end 151.2316 117.983) (width 2.2) (layer B.Cu) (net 1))
 (segment (start 153.4414 120.1928) (end 153.4414 120.3452) (width 2.2) (layer B.Cu) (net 1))
 (segment (start 151.2316 117.983) (end 153.4414 120.1928) (width 2.2) (layer B.Cu) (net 1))
 (segment (start 151.2316 124.0536) (end 151.2316 122.555) (width 2.2) (layer B.Cu) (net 1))
 (segment (start 151.2316 122.555) (end 153.4414 120.3452) (width 2.2) (layer B.Cu) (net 1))
 (segment (start 153.4414 120.3452) (end 153.5938 120.1928) (width 2.2) (layer B.Cu) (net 1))
 (segment (start 146.1516 124.0536) (end 146.1516 122.1486) (width 2.2) (layer B.Cu) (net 1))
 (segment (start 146.1516 122.1486) (end 148.1074 120.1928) (width 2.2) (layer B.Cu) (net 1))
 (segment (start 151.2316 122.4534) (end 151.2316 122.1486) (width 2.2) (layer B.Cu) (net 1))
 (segment (start 151.2316 122.1486) (end 149.2758 120.1928) (width 2.2) (layer B.Cu) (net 1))
 (segment (start 144.145 120.1928) (end 144.145 120.2182) (width 2.2) (layer B.Cu) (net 1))
 (segment (start 144.145 120.2182) (end 146.1516 122.2248) (width 2.2) (layer B.Cu) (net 1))
 (segment (start 138.5316 124.0536) (end 138.5316 122.5423) (width 2.2) (layer B.Cu) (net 1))
 (segment (start 140.8811 120.1928) (end 144.145 120.1928) (width 2.2) (layer B.Cu) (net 1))
 (segment (start 144.145 120.1928) (end 146.1008 120.1928) (width 2.2) (layer B.Cu) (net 1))
 (segment (start 138.5316 122.5423) (end 140.8811 120.1928) (width 2.2) (layer B.Cu) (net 1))
 (segment (start 157.6959 123.3297) (end 157.6959 122.8344) (width 2.2) (layer B.Cu) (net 1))
 (segment (start 157.6959 122.8344) (end 156.2481 121.3866) (width 2.2) (layer B.Cu) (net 1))
 (segment (start 157.6197 120.1928) (end 153.5938 120.1928) (width 2.2) (layer B.Cu) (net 1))
 (segment (start 153.5938 120.1928) (end 150.1902 120.1928) (width 2.2) (layer B.Cu) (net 1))
 (segment (start 150.1902 120.1928) (end 149.2758 120.1928) (width 2.2) (layer B.Cu) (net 1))
 (segment (start 149.2758 120.1928) (end 148.1074 120.1928) (width 2.2) (layer B.Cu) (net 1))
 (segment (start 148.1074 120.1928) (end 146.1008 120.1928) (width 2.2) (layer B.Cu) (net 1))
 (segment (start 148.0566 120.2436) (end 155.1051 120.2436) (width 2.2) (layer B.Cu) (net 1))
 (segment (start 156.2481 121.3866) (end 157.6197 121.3866) (width 2.2) (layer B.Cu) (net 1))
 (segment (start 155.1051 120.2436) (end 156.2481 121.3866) (width 2.2) (layer B.Cu) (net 1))
 (segment (start 151.2316 124.0536) (end 151.2316 130.8735) (width 2.2) (layer B.Cu) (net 1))
 (segment (start 149.8981 132.207) (end 148.5519 132.207) (width 2.2) (layer B.Cu) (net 1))
 (segment (start 151.2316 130.8735) (end 149.8981 132.207) (width 2.2) (layer B.Cu) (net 1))
 (segment (start 146.1516 124.0536) (end 146.1516 122.2248) (width 2.2) (layer B.Cu) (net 1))
 (segment (start 146.1516 122.2248) (end 146.1516 120.2436) (width 2.2) (layer B.Cu) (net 1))
 (segment (start 146.1516 120.2436) (end 146.1897 120.2817) (width 2.2) (layer B.Cu) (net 1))
 (segment (start 146.1897 120.2817) (end 146.1897 120.4341) (width 2.2) (layer B.Cu) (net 1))
 (segment (start 146.1897 120.4341) (end 146.1897 120.2436) (width 2.2) (layer B.Cu) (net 1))
 (segment (start 151.2316 122.4534) (end 151.2316 116.573598) (width 2.2) (layer B.Cu) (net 1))
 (segment (start 138.5316 120.2436) (end 146.1897 120.2436) (width 2.2) (layer B.Cu) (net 1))
 (segment (start 146.1897 120.2436) (end 148.0566 120.2436) (width 2.2) (layer B.Cu) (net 1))
 (segment (start 148.0566 120.2436) (end 151.0665 120.2436) (width 2.2) (layer B.Cu) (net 1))
 (segment (start 151.2316 120.4087) (end 151.2316 122.4534) (width 2.2) (layer B.Cu) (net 1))
 (segment (start 151.2316 122.4534) (end 151.2316 124.0536) (width 2.2) (layer B.Cu) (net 1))
 (segment (start 151.0665 120.2436) (end 151.2316 120.4087) (width 2.2) (layer B.Cu) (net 1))
 (segment (start 138.5316 124.0536) (end 138.5316 120.2436) (width 2.2) (layer B.Cu) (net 1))
 (segment (start 138.5316 120.2436) (end 138.5316 116.4336) (width 2.2) (layer B.Cu) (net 1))
 (segment (start 157.6197 120.1928) (end 157.6197 121.3866) (width 2.2) (layer B.Cu) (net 1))
 (segment (start 157.6197 121.3866) (end 157.6197 123.2535) (width 2.2) (layer B.Cu) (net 1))
 (segment (start 157.6197 123.2535) (end 157.6959 123.3297) (width 2.2) (layer B.Cu) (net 1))
 (segment (start 148.5519 132.207) (end 148.5519 132.5753) (width 2.2) (layer B.Cu) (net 1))
 (segment (start 147.4724 135.2804) (end 147.828 135.2804) (width 2.2) (layer B.Cu) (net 1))
 (segment (start 147.828 135.2804) (end 148.5519 134.5565) (width 2.2) (layer B.Cu) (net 1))
 (segment (start 148.5519 134.5565) (end 148.5519 132.207) (width 2.2) (layer B.Cu) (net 1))
 (segment (start 153.7716 116.4336) (end 153.7716 116.4209) (width 2.2) (layer B.Cu) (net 2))
 (segment (start 153.7716 116.4209) (end 154.9997 115.1928) (width 2.2) (layer B.Cu) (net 2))
 (segment (start 154.9997 115.1928) (end 157.6197 115.1928) (width 2.2) (layer B.Cu) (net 2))
 (segment (start 157.5981 115.2144) (end 157.6197 115.1928) (width 2.2) (layer B.Cu) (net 2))
 (segment (start 148.6916 124.0536) (end 148.6916 125.3744) (width 2.2) (layer B.Cu) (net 4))
 (segment (start 143.6116 124.0536) (end 143.6116 131.3434) (width 2.2) (layer B.Cu) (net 4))
 (segment (start 143.6116 131.3434) (end 143.5519 131.4031) (width 2.2) (layer B.Cu) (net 4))
 (segment (start 148.6916 125.3744) (end 148.6916 126.9238) (width 2.2) (layer B.Cu) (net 4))
 (segment (start 148.6916 126.9238) (end 146.3802 129.2352) (width 2.2) (layer B.Cu) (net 4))
 (segment (start 146.3802 129.2352) (end 145.7198 129.2352) (width 2.2) (layer B.Cu) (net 4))
 (segment (start 144.9324 135.2804) (end 143.4973 135.2804) (width 2.2) (layer B.Cu) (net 4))
 (segment (start 143.4973 135.2804) (end 143.5519 135.2258) (width 2.2) (layer B.Cu) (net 4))
 (segment (start 143.5519 135.2258) (end 143.5519 132.207) (width 2.2) (layer B.Cu) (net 4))
 (segment (start 143.5519 132.207) (end 143.5519 131.4031) (width 2.2) (layer B.Cu) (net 4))
 (segment (start 143.5519 131.4031) (end 145.7198 129.2352) (width 2.2) (layer B.Cu) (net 4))
 (segment (start 145.7198 129.2352) (end 148.6281 129.2352) (width 2.2) (layer B.Cu) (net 4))
 (segment (start 143.4973 135.2804) (end 143.5519 135.2258) (width 2.2) (layer B.Cu) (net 4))
 (segment (start 148.6916 125.3744) (end 148.6916 129.1717) (width 2.2) (layer B.Cu) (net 4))
 (segment (start 148.6916 129.1717) (end 148.6408 129.2225) (width 2.2) (layer B.Cu) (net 4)))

